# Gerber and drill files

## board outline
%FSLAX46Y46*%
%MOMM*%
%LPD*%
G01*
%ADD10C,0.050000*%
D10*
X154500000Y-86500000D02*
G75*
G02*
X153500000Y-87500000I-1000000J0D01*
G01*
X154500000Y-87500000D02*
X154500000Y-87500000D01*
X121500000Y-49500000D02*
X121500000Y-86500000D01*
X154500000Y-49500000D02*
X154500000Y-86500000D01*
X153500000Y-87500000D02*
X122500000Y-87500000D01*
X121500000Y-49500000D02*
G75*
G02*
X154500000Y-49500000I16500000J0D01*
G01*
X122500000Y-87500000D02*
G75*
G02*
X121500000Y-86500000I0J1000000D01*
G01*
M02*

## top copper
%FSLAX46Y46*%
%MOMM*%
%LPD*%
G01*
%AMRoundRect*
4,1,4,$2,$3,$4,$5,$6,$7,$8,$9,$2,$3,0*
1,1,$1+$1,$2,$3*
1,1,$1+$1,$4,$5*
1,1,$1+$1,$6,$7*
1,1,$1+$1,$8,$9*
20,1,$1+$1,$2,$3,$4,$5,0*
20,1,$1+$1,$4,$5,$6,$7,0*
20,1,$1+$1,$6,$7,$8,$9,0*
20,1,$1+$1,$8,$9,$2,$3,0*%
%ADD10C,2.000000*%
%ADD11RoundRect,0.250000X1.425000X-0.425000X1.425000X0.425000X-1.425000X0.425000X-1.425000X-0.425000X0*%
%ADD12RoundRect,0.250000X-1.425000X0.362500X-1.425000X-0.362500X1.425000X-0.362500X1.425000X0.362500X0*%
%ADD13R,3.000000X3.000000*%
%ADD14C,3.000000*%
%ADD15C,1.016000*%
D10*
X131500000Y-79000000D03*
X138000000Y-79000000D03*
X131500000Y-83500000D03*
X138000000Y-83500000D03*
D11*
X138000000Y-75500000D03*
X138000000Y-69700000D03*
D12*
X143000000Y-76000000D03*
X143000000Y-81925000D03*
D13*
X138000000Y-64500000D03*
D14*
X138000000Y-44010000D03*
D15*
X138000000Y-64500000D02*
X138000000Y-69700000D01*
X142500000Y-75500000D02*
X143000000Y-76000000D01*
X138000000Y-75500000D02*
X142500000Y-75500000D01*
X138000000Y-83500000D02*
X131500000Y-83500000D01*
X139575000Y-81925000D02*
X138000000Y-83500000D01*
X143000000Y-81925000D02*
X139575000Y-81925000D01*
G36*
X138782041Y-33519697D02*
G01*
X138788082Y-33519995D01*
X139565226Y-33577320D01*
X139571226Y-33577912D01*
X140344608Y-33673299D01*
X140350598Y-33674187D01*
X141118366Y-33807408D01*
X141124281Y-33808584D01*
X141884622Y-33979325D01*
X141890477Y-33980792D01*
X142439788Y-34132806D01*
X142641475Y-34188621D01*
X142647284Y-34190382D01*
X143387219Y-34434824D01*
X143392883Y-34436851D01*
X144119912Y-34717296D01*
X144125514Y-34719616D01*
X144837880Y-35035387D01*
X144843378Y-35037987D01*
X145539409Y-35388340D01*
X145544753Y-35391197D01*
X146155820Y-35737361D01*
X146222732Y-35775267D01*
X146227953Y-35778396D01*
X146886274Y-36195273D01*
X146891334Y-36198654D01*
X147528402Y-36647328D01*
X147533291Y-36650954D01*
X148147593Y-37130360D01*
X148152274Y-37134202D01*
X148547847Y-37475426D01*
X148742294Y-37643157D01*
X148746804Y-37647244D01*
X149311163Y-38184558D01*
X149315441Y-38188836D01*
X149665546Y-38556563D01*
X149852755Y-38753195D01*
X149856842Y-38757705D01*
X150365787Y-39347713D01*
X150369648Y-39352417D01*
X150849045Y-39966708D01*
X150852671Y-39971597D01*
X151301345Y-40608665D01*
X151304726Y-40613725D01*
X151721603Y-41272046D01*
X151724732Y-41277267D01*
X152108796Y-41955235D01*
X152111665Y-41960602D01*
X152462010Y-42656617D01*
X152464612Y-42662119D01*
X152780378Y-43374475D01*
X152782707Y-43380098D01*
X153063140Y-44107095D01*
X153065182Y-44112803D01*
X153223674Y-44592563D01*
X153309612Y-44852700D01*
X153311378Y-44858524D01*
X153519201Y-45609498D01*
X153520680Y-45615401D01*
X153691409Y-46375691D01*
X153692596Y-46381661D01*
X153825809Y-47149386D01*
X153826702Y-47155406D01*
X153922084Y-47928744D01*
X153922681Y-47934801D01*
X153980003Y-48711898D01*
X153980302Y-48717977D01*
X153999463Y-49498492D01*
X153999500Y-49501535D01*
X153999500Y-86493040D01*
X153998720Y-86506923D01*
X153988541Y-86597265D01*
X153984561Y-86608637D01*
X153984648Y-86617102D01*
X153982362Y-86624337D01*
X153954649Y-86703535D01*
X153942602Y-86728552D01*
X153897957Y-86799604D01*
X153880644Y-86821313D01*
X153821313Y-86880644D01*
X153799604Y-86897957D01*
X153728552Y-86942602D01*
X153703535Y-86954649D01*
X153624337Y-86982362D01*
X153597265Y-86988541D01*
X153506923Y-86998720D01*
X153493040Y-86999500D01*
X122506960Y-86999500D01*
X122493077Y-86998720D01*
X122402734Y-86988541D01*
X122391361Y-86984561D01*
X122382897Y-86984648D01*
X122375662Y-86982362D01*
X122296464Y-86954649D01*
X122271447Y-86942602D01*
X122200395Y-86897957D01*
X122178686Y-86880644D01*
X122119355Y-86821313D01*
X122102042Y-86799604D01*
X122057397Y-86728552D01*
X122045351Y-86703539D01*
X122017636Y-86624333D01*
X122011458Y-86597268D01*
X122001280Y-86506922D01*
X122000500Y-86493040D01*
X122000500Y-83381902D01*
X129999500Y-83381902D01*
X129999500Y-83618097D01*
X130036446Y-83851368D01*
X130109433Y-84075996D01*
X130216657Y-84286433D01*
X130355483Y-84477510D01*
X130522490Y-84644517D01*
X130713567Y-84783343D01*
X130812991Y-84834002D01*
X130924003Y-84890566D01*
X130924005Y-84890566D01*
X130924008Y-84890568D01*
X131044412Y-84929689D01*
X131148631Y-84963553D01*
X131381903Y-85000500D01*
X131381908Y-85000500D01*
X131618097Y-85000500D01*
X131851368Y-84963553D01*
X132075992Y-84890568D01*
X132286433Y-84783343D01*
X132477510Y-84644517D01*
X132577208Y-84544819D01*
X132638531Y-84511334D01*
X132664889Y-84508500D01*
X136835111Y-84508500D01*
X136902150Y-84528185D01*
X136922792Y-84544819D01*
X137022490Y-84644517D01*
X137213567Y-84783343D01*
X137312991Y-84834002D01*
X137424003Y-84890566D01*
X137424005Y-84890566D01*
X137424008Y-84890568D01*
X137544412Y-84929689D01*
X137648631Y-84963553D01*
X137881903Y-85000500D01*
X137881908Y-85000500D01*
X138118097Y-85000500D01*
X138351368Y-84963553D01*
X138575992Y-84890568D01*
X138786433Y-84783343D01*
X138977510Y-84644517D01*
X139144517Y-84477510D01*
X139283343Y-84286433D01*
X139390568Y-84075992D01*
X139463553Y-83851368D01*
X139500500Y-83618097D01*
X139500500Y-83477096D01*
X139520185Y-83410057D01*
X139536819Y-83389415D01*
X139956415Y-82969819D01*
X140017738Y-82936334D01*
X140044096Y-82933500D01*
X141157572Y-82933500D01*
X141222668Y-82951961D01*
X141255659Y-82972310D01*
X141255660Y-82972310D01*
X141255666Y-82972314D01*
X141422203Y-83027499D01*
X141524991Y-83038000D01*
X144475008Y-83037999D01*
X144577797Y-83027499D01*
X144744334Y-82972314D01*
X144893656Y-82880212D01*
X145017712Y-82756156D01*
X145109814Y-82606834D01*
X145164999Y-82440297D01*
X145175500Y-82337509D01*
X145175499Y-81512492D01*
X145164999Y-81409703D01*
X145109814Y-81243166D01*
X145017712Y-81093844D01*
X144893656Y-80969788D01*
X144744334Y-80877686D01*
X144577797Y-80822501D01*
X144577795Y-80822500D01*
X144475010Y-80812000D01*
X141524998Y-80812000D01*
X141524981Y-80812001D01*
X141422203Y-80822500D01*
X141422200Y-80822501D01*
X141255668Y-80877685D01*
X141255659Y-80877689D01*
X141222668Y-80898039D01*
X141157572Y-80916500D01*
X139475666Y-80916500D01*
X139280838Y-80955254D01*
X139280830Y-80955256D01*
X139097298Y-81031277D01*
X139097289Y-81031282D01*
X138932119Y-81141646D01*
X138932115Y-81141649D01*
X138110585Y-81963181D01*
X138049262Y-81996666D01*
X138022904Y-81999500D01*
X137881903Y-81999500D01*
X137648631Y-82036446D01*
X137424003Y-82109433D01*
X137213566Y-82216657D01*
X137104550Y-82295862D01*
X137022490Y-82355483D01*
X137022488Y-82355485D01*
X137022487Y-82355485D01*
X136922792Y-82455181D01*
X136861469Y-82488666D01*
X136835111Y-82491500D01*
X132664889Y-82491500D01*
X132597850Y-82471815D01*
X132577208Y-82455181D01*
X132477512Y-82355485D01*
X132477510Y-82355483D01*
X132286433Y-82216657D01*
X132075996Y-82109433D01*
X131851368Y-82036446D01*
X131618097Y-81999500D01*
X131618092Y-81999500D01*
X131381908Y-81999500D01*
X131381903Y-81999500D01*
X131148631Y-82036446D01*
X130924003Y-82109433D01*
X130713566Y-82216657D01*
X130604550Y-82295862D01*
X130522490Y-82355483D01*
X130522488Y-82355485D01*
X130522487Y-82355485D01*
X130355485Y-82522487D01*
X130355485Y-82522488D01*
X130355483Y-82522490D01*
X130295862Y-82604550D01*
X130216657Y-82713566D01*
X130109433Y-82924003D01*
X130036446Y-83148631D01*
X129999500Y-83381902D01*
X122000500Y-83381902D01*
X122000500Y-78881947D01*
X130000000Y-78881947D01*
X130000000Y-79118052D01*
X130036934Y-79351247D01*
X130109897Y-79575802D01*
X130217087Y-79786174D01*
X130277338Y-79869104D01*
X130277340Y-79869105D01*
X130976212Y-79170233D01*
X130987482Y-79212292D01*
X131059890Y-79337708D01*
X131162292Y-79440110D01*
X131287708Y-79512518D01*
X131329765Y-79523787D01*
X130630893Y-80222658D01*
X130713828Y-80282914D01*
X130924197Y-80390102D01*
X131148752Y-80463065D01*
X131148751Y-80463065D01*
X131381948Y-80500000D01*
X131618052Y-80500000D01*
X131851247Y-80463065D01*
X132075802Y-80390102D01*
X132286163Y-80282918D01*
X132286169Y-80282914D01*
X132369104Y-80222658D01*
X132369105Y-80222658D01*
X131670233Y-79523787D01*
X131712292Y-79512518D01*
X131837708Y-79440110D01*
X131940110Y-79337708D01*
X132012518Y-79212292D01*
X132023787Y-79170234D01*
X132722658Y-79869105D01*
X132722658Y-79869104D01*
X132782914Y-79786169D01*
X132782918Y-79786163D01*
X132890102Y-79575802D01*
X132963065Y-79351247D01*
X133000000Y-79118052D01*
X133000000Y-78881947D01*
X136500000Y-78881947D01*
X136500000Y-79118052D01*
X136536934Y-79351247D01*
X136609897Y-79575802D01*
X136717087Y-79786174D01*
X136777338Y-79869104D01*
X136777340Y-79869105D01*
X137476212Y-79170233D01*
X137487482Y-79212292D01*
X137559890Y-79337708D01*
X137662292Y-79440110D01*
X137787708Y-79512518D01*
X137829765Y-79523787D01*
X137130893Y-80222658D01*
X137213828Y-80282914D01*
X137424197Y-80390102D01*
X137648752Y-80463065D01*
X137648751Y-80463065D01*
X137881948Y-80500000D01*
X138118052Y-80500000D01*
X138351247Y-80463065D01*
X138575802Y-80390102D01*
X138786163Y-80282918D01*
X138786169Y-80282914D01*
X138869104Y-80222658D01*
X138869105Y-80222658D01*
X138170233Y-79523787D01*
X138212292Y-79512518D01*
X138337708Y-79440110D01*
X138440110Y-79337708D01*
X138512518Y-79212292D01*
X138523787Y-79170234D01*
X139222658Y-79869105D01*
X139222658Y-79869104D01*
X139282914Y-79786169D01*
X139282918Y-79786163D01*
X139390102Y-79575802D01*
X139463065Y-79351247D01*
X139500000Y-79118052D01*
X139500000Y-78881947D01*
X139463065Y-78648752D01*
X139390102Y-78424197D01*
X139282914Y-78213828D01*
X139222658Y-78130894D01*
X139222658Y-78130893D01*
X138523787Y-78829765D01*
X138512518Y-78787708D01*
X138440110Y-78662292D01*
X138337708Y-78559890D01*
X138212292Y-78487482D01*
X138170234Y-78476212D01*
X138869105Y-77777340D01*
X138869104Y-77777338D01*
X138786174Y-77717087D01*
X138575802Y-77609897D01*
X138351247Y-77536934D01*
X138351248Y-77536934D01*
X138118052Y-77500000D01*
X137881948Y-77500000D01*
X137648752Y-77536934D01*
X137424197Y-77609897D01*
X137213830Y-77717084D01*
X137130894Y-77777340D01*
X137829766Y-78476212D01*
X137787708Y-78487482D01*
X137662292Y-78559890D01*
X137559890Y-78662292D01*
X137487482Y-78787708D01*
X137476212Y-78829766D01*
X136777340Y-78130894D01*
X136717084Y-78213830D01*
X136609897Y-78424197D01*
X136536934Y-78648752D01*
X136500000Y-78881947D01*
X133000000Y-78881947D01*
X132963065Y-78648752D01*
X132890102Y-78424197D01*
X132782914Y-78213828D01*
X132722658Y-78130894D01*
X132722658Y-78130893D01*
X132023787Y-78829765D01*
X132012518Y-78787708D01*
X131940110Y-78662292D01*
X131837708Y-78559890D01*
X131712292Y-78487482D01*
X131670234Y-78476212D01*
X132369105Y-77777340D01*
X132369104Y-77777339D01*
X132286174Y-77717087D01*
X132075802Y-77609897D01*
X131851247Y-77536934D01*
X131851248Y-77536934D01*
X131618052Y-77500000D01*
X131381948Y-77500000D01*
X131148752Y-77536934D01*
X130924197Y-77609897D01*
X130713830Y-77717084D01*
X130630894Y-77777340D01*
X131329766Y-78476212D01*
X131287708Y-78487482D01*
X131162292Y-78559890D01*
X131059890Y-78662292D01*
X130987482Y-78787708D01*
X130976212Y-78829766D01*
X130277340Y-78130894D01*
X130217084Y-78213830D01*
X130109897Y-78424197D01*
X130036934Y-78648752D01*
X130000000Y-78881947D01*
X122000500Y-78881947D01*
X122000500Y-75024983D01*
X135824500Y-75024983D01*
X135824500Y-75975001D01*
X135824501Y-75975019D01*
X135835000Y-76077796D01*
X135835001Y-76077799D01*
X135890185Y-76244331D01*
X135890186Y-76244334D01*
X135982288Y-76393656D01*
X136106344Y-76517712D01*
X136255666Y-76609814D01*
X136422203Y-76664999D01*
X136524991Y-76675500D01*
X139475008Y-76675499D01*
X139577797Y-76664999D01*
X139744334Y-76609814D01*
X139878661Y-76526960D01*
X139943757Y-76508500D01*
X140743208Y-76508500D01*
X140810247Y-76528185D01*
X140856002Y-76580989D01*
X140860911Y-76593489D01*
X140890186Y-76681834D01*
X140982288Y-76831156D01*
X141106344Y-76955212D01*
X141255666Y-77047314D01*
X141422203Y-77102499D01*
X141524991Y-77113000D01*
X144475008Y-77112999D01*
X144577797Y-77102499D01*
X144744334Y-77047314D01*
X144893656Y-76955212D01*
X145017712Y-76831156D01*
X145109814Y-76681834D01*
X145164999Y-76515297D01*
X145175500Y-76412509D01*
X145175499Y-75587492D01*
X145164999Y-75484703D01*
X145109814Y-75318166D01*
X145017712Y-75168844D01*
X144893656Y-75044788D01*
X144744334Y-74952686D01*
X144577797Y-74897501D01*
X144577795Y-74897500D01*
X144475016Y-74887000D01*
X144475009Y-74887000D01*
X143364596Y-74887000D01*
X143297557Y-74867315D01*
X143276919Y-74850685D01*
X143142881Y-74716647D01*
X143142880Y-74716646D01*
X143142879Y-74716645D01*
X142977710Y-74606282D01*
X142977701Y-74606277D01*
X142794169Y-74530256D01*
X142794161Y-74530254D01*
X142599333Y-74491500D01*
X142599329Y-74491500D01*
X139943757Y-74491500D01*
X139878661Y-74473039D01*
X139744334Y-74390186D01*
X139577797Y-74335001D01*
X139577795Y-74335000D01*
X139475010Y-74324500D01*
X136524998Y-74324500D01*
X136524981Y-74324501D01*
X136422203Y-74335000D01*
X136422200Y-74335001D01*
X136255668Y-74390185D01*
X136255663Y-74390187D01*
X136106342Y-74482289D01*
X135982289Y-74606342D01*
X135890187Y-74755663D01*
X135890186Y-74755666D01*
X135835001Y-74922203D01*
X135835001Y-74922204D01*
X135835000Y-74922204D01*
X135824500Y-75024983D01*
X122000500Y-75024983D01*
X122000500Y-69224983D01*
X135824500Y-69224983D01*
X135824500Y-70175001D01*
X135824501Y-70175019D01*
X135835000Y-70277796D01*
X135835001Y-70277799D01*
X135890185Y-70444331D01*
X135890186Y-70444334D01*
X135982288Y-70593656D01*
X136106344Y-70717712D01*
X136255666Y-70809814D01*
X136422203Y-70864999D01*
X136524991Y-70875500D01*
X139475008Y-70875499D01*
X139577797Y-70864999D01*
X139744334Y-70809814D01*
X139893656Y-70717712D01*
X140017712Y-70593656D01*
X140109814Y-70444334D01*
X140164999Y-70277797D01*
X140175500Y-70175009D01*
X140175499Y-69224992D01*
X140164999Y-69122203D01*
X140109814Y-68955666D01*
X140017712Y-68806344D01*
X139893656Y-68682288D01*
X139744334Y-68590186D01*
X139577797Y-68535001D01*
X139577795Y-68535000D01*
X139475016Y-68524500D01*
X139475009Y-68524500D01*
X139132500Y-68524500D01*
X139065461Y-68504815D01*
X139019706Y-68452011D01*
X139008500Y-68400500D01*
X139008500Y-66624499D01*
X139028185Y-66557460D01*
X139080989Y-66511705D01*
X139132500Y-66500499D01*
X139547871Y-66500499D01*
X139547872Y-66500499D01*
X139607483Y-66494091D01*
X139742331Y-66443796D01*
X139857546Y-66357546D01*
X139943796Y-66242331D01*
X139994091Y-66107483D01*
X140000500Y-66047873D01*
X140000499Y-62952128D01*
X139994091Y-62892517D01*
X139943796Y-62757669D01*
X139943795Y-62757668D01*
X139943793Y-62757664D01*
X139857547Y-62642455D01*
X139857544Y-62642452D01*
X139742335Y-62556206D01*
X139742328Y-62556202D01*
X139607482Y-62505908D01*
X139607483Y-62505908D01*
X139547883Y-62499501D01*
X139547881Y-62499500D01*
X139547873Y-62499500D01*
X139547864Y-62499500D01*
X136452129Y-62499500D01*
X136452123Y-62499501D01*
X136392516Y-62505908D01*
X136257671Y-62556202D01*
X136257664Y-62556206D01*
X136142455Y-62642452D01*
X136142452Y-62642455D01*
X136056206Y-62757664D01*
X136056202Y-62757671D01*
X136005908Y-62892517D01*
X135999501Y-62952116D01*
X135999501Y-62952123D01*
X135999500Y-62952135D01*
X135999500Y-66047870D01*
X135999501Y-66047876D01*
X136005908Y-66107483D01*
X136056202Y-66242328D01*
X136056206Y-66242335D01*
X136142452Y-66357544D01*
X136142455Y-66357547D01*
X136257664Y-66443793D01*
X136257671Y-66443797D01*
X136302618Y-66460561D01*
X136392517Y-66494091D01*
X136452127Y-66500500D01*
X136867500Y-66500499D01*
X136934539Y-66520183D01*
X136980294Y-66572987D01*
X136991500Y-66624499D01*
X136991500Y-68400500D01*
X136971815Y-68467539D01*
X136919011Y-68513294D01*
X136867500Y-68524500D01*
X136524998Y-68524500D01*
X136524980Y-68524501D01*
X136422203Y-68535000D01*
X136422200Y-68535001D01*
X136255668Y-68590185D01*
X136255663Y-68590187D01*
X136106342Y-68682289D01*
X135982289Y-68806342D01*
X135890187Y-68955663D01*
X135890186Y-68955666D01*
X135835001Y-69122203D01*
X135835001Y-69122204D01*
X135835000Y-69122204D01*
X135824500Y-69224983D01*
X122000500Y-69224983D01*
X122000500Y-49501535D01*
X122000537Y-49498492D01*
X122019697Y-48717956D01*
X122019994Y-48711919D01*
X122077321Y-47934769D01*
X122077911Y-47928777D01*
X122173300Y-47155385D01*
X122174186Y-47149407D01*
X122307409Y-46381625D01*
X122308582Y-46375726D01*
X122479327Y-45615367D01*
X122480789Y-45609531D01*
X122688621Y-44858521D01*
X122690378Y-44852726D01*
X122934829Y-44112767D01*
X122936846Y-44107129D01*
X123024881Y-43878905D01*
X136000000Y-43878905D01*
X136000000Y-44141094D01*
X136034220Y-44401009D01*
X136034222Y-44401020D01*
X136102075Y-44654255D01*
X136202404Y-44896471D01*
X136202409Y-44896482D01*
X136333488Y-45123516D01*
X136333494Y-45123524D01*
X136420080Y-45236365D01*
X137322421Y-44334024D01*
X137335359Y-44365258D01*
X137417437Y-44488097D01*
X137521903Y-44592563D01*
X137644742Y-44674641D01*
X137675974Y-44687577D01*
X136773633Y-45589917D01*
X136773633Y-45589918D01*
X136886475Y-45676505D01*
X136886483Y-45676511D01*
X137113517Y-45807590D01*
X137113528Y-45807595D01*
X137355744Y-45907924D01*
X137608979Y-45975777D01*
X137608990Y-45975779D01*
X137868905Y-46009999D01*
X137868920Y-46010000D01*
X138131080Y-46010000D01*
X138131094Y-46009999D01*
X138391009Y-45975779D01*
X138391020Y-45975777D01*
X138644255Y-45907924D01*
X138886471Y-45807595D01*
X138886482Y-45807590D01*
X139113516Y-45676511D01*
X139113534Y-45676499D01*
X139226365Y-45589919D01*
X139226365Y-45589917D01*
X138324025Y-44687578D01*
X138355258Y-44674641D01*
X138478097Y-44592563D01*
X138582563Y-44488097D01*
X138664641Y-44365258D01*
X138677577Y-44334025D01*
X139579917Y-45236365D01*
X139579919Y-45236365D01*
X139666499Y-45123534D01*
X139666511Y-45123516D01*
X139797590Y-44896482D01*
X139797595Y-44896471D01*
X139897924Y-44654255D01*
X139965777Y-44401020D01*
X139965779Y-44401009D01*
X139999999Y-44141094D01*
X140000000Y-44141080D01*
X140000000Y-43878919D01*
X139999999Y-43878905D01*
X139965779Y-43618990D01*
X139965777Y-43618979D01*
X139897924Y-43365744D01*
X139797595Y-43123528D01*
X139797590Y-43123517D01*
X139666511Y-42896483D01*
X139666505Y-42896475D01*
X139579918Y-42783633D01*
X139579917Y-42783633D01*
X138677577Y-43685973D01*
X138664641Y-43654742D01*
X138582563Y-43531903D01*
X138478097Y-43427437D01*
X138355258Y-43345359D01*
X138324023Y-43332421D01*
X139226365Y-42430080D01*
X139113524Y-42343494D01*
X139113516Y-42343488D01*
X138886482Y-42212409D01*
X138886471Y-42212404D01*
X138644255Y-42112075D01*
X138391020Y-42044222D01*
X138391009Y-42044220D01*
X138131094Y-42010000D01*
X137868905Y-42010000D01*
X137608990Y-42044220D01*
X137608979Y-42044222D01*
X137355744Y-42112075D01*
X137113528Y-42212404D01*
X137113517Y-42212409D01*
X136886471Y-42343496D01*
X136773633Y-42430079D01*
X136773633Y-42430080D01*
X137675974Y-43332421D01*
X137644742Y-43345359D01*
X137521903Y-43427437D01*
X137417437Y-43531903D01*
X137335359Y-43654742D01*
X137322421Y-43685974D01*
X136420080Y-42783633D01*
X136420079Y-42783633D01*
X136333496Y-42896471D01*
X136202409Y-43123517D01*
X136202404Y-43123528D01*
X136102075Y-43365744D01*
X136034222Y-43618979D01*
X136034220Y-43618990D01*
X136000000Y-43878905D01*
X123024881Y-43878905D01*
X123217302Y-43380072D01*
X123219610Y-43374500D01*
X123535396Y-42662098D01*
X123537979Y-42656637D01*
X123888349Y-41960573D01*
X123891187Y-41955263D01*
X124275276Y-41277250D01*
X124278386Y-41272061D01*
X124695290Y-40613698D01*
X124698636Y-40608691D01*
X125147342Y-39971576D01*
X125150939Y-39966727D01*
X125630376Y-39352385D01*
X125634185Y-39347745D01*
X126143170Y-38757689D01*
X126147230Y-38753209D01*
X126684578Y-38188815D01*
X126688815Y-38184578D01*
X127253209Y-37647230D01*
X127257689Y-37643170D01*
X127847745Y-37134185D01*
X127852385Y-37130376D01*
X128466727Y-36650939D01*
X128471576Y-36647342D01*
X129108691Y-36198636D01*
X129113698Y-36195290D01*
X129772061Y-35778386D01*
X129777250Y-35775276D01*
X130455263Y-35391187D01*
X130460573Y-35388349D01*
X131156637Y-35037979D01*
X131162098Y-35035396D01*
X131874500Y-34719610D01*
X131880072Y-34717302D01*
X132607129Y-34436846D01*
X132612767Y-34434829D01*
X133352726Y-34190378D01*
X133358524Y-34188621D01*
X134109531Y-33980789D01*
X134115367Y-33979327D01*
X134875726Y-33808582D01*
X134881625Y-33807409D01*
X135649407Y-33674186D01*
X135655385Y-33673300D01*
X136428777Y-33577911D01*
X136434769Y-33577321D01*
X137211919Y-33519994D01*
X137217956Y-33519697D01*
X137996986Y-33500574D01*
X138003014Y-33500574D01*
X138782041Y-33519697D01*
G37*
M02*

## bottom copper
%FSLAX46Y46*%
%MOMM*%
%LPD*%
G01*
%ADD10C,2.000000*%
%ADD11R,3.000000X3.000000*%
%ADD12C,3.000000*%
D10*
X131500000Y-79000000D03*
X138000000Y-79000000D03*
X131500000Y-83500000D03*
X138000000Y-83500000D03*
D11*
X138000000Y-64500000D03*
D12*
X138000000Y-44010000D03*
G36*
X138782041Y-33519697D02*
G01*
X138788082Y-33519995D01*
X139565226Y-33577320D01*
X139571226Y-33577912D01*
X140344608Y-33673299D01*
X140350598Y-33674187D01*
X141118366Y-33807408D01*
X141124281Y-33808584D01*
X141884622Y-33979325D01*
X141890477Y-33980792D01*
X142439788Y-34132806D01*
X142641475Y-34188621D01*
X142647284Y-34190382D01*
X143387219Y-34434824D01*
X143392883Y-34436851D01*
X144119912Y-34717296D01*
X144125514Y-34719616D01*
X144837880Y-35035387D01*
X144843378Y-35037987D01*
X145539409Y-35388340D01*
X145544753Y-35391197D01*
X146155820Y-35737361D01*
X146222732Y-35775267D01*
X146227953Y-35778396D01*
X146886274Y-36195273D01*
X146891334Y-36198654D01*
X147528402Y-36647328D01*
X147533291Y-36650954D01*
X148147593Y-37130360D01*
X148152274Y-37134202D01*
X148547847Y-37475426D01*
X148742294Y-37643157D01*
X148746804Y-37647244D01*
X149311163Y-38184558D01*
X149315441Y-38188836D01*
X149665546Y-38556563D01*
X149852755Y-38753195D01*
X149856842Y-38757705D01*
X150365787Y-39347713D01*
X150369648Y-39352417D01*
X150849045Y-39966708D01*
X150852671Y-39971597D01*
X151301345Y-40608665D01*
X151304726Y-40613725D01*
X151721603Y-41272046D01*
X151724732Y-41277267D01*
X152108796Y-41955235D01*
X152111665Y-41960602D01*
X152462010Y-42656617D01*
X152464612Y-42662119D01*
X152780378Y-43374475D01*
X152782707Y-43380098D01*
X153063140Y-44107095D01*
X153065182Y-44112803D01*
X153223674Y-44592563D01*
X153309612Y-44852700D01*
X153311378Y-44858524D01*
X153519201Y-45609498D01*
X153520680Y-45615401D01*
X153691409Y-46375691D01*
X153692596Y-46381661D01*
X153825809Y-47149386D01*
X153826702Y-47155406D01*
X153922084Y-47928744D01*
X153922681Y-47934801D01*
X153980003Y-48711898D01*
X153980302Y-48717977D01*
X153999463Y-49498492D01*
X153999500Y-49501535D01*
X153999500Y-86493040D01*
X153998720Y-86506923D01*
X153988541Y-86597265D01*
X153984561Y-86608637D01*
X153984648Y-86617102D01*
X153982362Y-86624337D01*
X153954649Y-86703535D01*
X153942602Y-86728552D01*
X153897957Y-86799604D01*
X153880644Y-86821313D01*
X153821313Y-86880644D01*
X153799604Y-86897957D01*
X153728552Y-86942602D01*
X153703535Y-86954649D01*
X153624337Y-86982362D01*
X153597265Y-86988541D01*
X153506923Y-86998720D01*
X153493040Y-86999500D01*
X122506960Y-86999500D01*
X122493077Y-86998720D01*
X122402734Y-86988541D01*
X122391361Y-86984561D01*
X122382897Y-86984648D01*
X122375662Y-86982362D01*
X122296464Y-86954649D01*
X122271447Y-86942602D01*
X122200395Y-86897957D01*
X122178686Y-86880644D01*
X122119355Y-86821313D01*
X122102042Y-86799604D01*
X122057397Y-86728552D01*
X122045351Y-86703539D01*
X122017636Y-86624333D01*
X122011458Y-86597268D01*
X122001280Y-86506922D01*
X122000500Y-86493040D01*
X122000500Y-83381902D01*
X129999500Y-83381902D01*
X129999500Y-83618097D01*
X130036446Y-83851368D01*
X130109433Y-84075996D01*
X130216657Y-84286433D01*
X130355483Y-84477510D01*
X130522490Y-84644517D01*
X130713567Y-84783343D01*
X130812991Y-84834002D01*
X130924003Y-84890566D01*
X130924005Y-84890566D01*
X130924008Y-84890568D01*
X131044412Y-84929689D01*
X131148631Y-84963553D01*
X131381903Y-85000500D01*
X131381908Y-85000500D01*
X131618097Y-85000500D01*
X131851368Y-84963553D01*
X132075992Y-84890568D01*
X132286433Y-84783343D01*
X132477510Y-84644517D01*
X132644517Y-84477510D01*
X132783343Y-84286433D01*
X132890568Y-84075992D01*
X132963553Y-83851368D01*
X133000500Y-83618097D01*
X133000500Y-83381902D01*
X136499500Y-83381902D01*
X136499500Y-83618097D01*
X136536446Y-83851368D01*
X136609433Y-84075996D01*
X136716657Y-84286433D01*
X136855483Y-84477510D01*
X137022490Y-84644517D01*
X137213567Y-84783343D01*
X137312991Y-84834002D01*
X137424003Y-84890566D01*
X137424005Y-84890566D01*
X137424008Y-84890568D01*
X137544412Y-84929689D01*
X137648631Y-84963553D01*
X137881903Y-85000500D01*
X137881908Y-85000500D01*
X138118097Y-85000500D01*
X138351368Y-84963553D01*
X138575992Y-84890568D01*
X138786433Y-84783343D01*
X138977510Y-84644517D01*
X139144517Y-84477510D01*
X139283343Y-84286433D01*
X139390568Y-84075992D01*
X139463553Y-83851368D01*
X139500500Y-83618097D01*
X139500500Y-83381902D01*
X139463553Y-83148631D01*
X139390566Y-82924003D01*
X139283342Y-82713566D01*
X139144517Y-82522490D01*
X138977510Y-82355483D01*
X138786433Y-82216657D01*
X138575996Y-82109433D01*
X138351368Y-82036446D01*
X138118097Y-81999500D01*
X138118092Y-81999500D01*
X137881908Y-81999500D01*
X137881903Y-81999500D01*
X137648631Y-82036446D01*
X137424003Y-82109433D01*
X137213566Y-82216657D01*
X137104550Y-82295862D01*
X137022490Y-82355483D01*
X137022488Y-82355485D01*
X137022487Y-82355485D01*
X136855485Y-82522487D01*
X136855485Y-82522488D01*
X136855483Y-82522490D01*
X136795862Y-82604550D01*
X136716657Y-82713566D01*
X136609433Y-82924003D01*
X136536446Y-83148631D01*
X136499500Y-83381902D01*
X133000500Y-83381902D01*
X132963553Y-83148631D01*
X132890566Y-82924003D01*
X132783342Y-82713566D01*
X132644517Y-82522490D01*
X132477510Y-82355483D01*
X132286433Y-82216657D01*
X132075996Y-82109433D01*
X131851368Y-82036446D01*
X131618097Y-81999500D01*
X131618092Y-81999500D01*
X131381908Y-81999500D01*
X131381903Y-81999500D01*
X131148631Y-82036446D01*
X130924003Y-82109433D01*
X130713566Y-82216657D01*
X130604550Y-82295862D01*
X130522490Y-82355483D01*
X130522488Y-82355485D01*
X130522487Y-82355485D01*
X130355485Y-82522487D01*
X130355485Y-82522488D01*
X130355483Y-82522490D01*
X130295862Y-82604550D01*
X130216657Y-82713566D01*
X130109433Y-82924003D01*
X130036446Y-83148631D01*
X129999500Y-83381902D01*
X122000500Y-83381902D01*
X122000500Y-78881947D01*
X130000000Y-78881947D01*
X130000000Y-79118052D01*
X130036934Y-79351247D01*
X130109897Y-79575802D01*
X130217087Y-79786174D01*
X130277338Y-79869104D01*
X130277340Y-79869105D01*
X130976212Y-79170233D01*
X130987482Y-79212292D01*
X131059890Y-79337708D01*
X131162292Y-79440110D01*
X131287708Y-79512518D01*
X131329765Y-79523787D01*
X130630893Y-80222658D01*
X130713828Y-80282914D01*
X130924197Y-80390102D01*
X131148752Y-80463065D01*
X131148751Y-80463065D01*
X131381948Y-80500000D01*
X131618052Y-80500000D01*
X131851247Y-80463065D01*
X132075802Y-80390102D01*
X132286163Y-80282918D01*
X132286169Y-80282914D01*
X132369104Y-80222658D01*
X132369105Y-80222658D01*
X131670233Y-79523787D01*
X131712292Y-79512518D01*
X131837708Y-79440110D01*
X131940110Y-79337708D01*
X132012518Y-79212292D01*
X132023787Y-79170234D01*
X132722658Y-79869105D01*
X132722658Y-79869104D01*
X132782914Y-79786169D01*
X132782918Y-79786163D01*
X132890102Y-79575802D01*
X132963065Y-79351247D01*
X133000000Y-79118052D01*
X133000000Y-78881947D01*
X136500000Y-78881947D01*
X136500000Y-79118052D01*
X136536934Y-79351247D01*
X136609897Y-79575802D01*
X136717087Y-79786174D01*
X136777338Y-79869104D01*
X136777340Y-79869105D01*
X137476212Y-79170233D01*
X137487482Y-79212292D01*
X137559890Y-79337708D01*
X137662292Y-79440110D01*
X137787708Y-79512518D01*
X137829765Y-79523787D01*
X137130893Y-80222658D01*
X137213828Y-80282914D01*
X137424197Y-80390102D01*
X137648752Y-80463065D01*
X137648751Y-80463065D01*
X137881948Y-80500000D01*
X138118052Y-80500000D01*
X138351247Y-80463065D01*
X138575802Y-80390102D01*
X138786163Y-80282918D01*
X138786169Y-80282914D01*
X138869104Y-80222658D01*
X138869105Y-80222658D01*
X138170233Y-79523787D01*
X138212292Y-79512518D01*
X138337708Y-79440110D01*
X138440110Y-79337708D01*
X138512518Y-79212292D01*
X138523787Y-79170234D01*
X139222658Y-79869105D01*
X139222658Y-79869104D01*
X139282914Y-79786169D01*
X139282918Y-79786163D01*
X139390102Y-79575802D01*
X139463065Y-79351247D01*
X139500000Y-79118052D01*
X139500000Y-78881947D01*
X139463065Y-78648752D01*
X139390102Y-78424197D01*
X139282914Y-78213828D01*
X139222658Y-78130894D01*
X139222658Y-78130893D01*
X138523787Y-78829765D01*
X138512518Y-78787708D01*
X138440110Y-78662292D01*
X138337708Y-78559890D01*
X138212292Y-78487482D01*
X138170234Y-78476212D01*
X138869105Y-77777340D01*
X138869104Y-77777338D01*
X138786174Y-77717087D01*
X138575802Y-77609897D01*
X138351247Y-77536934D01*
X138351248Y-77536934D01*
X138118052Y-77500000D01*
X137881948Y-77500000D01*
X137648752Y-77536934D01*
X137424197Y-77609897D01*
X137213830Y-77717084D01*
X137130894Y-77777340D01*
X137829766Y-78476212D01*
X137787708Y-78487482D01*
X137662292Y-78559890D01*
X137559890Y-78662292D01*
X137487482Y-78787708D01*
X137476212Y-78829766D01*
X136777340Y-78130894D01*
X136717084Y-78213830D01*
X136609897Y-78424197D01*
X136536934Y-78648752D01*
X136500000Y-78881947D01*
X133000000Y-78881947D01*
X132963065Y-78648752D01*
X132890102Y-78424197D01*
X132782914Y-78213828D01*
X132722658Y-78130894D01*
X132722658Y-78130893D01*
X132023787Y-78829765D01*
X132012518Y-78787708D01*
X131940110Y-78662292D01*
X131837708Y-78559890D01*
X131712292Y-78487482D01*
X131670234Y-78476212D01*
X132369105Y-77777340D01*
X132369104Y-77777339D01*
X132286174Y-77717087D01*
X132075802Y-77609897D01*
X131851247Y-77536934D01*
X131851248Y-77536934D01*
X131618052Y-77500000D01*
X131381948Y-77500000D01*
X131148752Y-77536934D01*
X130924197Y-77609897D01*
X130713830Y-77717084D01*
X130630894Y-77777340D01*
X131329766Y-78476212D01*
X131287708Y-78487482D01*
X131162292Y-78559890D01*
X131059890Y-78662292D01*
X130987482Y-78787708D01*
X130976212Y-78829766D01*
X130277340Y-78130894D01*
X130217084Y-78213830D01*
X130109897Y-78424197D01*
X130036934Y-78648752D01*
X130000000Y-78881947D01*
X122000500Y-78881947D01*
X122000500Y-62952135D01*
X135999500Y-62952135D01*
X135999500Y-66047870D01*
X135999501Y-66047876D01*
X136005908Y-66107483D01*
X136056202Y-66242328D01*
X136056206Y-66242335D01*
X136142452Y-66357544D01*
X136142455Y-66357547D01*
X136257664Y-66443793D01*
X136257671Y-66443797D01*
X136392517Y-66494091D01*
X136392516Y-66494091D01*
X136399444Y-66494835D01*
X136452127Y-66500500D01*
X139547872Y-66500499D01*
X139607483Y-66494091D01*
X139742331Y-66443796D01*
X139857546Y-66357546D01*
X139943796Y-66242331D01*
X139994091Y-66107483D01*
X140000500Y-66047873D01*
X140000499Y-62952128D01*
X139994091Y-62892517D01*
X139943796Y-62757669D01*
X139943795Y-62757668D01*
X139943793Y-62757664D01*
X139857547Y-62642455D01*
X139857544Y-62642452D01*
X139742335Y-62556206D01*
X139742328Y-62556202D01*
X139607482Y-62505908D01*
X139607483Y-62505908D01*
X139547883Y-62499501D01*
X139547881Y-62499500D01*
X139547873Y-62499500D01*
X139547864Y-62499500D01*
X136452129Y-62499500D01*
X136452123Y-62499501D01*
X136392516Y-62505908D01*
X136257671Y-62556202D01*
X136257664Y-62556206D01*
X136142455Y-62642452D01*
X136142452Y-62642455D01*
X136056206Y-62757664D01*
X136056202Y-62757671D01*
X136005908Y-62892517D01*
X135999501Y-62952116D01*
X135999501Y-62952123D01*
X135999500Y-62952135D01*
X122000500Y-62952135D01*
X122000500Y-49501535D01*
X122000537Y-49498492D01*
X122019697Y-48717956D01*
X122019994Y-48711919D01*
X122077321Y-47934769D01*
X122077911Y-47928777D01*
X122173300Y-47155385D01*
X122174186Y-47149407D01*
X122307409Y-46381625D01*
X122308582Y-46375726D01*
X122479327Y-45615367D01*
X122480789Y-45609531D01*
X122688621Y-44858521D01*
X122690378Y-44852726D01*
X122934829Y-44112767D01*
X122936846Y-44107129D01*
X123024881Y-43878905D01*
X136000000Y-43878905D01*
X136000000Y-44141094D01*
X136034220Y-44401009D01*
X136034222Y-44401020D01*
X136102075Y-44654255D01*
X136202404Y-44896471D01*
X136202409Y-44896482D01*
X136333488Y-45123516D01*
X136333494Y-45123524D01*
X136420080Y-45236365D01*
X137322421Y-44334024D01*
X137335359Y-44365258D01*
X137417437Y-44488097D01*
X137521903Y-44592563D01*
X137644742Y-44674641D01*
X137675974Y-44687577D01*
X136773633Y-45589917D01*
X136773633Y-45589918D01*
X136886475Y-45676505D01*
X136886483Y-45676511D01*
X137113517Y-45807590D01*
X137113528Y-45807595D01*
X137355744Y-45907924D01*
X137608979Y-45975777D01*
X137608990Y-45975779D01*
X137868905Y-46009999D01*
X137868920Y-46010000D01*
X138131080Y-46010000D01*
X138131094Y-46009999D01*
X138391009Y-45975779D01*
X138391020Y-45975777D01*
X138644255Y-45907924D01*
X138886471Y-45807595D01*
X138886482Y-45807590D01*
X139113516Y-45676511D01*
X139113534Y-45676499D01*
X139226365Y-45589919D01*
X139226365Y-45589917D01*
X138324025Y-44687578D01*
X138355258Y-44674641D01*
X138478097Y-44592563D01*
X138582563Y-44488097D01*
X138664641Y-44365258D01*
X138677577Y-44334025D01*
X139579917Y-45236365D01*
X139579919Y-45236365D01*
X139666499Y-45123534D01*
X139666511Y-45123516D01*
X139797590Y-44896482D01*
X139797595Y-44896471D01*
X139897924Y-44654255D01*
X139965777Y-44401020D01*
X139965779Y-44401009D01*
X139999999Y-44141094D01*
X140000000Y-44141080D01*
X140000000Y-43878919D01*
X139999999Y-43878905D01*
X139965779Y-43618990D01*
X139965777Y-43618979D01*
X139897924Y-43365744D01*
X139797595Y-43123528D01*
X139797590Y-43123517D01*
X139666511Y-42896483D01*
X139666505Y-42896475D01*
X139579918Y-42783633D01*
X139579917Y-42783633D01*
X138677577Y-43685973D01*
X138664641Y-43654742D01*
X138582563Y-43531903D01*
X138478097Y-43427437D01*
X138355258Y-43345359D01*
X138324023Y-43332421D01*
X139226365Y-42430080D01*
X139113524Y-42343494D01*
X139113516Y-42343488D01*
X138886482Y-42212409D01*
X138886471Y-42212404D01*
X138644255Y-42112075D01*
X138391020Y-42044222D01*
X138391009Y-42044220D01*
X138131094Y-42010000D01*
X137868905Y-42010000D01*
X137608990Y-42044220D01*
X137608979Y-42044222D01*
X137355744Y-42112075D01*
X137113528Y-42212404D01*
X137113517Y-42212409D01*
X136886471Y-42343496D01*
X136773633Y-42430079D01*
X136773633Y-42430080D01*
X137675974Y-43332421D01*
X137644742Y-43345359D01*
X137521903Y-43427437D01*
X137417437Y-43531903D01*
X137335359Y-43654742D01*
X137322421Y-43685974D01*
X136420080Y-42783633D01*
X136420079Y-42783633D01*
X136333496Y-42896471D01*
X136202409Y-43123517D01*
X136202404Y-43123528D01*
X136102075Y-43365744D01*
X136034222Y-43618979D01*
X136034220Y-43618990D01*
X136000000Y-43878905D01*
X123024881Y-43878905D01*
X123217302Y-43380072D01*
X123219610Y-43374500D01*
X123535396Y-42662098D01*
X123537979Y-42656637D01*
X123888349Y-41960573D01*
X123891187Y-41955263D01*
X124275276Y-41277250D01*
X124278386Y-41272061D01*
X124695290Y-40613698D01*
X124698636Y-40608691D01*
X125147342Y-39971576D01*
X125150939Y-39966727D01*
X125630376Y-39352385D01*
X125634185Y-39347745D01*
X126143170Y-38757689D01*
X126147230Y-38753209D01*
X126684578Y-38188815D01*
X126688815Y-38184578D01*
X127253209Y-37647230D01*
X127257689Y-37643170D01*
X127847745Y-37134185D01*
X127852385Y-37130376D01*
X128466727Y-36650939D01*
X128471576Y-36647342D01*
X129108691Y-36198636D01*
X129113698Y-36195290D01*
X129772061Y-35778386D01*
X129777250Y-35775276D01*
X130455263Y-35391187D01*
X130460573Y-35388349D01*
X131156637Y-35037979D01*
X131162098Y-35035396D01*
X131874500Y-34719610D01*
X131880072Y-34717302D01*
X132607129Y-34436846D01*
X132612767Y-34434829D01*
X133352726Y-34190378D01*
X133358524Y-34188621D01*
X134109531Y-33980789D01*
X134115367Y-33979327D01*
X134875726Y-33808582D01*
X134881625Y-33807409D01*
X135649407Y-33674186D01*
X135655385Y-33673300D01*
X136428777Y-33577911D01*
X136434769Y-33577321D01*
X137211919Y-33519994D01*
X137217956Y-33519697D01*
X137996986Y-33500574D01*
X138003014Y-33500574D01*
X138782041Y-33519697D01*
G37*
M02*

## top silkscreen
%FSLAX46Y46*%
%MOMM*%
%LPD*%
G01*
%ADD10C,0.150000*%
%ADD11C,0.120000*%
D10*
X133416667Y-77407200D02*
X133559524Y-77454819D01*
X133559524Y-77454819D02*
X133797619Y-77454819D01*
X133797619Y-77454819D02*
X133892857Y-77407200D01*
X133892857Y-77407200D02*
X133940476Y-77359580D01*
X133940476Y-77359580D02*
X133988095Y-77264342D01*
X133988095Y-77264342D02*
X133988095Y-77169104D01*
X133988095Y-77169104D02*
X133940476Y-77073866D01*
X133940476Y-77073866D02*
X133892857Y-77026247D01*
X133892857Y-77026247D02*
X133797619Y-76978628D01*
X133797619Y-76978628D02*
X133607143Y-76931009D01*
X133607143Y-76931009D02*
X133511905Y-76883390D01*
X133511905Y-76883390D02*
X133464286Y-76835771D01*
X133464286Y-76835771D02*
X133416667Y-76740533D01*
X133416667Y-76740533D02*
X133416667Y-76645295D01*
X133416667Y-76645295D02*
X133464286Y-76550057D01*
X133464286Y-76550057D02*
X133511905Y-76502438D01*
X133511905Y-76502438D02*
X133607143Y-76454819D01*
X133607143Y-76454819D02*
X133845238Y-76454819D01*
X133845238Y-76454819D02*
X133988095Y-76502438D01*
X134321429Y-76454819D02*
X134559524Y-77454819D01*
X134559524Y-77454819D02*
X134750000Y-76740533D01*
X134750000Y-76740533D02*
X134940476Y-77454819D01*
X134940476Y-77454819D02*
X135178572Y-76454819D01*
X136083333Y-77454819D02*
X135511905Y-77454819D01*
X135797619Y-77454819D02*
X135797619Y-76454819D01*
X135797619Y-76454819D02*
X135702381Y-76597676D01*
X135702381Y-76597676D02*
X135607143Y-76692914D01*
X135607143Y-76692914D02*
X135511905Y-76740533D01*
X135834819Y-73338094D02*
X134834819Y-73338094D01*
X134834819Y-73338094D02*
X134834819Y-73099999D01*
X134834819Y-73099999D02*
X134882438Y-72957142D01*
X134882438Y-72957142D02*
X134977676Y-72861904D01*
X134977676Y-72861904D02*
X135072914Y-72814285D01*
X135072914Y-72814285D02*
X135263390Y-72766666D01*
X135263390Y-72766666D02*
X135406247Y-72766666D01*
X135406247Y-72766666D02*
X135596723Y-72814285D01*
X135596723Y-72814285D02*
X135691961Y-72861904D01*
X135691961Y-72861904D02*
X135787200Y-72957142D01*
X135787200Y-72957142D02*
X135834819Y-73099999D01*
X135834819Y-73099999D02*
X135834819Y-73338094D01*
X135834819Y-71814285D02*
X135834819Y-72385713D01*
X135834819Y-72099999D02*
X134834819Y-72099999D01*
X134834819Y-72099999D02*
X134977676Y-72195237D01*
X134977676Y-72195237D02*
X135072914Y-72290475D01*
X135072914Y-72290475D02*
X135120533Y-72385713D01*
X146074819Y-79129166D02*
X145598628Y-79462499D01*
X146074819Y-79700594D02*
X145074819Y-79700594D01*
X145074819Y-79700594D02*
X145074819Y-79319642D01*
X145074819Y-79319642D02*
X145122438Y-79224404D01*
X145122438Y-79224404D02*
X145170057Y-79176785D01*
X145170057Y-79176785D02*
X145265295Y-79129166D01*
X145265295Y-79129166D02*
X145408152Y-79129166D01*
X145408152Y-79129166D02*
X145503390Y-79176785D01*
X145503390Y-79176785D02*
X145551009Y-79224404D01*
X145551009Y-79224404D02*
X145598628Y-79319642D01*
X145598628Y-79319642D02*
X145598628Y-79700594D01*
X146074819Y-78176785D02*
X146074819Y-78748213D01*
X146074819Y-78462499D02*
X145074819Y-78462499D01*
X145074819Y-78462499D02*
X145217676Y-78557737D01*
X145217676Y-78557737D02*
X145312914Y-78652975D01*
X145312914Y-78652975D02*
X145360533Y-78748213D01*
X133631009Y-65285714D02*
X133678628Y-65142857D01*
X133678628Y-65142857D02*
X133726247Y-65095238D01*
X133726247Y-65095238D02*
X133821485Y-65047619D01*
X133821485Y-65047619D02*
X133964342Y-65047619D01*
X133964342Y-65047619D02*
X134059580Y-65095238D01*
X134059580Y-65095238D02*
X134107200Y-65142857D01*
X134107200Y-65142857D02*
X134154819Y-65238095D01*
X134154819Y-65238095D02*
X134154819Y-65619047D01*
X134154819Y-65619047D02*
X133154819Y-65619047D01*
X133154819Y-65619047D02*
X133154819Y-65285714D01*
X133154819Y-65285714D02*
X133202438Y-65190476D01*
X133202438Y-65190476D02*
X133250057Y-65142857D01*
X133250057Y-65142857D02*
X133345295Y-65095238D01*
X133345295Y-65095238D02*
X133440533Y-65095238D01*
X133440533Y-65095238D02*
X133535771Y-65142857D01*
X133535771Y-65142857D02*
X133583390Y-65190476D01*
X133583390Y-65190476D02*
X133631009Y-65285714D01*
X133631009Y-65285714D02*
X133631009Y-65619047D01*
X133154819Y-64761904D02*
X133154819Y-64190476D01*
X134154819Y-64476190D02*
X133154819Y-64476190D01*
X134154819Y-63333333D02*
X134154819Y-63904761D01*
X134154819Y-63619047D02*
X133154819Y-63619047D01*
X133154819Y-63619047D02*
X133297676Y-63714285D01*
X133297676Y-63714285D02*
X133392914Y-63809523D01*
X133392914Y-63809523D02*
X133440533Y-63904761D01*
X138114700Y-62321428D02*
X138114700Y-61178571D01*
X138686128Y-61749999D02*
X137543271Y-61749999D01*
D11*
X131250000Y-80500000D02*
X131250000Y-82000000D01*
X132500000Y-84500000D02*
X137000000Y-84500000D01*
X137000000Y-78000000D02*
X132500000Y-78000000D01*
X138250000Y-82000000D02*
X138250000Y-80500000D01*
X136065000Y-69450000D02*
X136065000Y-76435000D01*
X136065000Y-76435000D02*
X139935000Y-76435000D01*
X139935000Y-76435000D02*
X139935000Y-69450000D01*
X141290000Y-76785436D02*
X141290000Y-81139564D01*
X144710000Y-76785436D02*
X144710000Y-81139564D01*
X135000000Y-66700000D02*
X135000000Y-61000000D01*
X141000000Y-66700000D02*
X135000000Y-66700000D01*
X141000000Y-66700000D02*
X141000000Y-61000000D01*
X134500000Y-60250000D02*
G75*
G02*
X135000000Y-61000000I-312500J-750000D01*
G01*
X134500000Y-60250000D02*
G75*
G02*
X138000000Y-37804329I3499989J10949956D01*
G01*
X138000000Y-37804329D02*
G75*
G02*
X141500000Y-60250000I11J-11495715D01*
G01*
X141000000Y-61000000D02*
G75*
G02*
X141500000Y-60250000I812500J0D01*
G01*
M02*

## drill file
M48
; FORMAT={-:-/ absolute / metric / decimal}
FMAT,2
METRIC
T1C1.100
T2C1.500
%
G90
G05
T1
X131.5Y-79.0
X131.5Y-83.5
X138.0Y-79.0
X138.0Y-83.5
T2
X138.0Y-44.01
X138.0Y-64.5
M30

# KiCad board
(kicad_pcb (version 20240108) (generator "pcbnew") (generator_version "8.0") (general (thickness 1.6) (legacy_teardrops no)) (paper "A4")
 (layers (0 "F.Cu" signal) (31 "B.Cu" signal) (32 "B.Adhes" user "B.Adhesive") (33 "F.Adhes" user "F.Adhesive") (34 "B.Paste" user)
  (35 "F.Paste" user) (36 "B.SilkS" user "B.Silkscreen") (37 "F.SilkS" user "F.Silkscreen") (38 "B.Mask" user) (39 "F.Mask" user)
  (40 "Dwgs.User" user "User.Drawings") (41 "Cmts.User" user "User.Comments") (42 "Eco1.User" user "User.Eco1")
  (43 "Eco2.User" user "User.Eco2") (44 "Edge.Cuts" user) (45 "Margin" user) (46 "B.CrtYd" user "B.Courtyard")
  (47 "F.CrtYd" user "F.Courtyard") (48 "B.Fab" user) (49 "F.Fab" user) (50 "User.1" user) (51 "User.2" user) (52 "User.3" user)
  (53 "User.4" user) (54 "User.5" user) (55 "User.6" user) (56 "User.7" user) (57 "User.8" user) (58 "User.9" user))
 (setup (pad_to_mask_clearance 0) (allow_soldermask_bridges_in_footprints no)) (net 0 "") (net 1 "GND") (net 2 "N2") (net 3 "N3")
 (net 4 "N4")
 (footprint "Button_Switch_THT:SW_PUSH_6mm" (layer "F.Cu") (at 131.5 79)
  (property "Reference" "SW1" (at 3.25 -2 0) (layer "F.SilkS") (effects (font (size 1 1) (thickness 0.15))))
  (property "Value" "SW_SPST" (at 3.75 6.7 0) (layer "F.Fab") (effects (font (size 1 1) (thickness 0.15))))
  (fp_line (start -0.25 1.5) (end -0.25 3) (stroke (width 0.12) (type solid)) (layer "F.SilkS"))
  (fp_line (start 1 5.5) (end 5.5 5.5) (stroke (width 0.12) (type solid)) (layer "F.SilkS"))
  (fp_line (start 5.5 -1) (end 1 -1) (stroke (width 0.12) (type solid)) (layer "F.SilkS"))
  (fp_line (start 6.75 3) (end 6.75 1.5) (stroke (width 0.12) (type solid)) (layer "F.SilkS"))
  (pad "1" thru_hole circle (at 0 0 90) (size 2 2) (drill 1.1) (layers "*.Cu" "*.Mask") (remove_unused_layers no) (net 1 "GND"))
  (pad "1" thru_hole circle (at 6.5 0 90) (size 2 2) (drill 1.1) (layers "*.Cu" "*.Mask") (remove_unused_layers no) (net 1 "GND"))
  (pad "2" thru_hole circle (at 0 4.5 90) (size 2 2) (drill 1.1) (layers "*.Cu" "*.Mask") (remove_unused_layers no) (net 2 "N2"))
  (pad "2" thru_hole circle (at 6.5 4.5 90) (size 2 2) (drill 1.1) (layers "*.Cu" "*.Mask") (remove_unused_layers no) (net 2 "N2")))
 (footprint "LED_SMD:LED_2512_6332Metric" (layer "F.Cu") (at 138 72.6 90)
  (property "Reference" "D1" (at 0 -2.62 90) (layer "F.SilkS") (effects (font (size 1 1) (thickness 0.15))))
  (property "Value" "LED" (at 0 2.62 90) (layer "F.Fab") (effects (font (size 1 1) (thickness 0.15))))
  (fp_line (start 3.15 -1.935) (end -3.835 -1.935) (stroke (width 0.12) (type solid)) (layer "F.SilkS"))
  (fp_line (start -3.835 -1.935) (end -3.835 1.935) (stroke (width 0.12) (type solid)) (layer "F.SilkS"))
  (fp_line (start -3.835 1.935) (end 3.15 1.935) (stroke (width 0.12) (type solid)) (layer "F.SilkS"))
  (pad "1" smd roundrect (at -2.9 0 90) (size 1.35 3.35) (layers "F.Cu" "F.Paste" "F.Mask") (roundrect_rratio 0.185185) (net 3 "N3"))
  (pad "2" smd roundrect (at 2.9 0 90) (size 1.35 3.35) (layers "F.Cu" "F.Paste" "F.Mask") (roundrect_rratio 0.185185) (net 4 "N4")))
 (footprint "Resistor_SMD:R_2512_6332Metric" (layer "F.Cu") (at 143 78.9625 -90)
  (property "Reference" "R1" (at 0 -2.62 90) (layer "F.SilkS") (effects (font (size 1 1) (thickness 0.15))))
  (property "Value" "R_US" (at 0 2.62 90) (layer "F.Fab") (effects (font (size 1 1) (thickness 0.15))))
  (fp_line (start -2.177064 1.71) (end 2.177064 1.71) (stroke (width 0.12) (type solid)) (layer "F.SilkS"))
  (fp_line (start -2.177064 -1.71) (end 2.177064 -1.71) (stroke (width 0.12) (type solid)) (layer "F.SilkS"))
  (pad "1" smd roundrect (at -2.9625 0 270) (size 1.225 3.35) (layers "F.Cu" "F.Paste" "F.Mask") (roundrect_rratio 0.204082) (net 3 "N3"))
  (pad "2" smd roundrect (at 2.9625 0 270) (size 1.225 3.35) (layers "F.Cu" "F.Paste" "F.Mask") (roundrect_rratio 0.204082) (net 2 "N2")))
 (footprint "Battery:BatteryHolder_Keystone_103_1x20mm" (layer "F.Cu") (at 138 64.5 90)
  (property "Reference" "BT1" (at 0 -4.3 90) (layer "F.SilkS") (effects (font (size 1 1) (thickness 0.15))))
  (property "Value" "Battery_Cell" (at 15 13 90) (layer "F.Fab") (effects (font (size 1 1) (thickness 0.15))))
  (fp_line (start -2.2 -3) (end 3.5 -3) (stroke (width 0.12) (type solid)) (layer "F.SilkS"))
  (fp_line (start -2.2 3) (end -2.2 -3) (stroke (width 0.12) (type solid)) (layer "F.SilkS"))
  (fp_line (start -2.2 3) (end 3.5 3) (stroke (width 0.12) (type solid)) (layer "F.SilkS"))
  (fp_arc (start 4.25 -3.5) (mid 3.950694 -3.136459) (end 3.5 -3) (stroke (width 0.12) (type solid)) (layer "F.SilkS"))
  (fp_arc (start 4.25 -3.5) (mid 16.971103 -11.358466) (end 26.695671 0) (stroke (width 0.12) (type solid)) (layer "F.SilkS"))
  (fp_arc (start 26.695671 0) (mid 16.971103 11.358466) (end 4.25 3.5) (stroke (width 0.12) (type solid)) (layer "F.SilkS"))
  (fp_arc (start 3.5 3) (mid 3.950694 3.136459) (end 4.25 3.5) (stroke (width 0.12) (type solid)) (layer "F.SilkS"))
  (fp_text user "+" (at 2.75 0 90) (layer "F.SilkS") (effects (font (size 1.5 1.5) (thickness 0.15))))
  (pad "1" thru_hole rect (at 0 0 90) (size 3 3) (drill 1.5) (layers "*.Cu" "*.Mask") (remove_unused_layers no) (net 4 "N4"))
  (pad "2" thru_hole circle (at 20.49 0 90) (size 3 3) (drill 1.5) (layers "*.Cu" "*.Mask") (remove_unused_layers no) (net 1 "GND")))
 (gr_arc (start 154.5 86.5) (mid 154.207107 87.207107) (end 153.5 87.5) (stroke (width 0.05) (type default)) (layer "Edge.Cuts"))
 (gr_line (start 154.5 87.5) (end 154.5 87.5) (stroke (width 0.05) (type default)) (layer "Edge.Cuts"))
 (gr_line (start 121.5 49.5) (end 121.5 86.5) (stroke (width 0.05) (type default)) (layer "Edge.Cuts"))
 (gr_line (start 154.5 49.5) (end 154.5 86.5) (stroke (width 0.05) (type default)) (layer "Edge.Cuts"))
 (gr_line (start 153.5 87.5) (end 122.5 87.5) (stroke (width 0.05) (type default)) (layer "Edge.Cuts"))
 (gr_arc (start 121.5 49.5) (mid 138 33) (end 154.5 49.5) (stroke (width 0.05) (type default)) (layer "Edge.Cuts"))
 (gr_arc (start 122.5 87.5) (mid 121.792893 87.207107) (end 121.5 86.5) (stroke (width 0.05) (type default)) (layer "Edge.Cuts"))
 (segment (start 138 64.5) (end 138 69.7) (width 1.016) (layer "F.Cu") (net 4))
 (segment (start 142.5 75.5) (end 143 76) (width 1.016) (layer "F.Cu") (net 3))
 (segment (start 138 75.5) (end 142.5 75.5) (width 1.016) (layer "F.Cu") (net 3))
 (segment (start 138 83.5) (end 131.5 83.5) (width 1.016) (layer "F.Cu") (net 2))
 (segment (start 139.575 81.925) (end 138 83.5) (width 1.016) (layer "F.Cu") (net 2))
 (segment (start 143 81.925) (end 139.575 81.925) (width 1.016) (layer "F.Cu") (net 2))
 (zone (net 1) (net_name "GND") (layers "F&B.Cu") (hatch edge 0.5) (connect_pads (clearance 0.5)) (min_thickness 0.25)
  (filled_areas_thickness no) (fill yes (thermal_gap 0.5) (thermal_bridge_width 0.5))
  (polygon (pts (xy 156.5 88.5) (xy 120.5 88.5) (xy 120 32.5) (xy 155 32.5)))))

